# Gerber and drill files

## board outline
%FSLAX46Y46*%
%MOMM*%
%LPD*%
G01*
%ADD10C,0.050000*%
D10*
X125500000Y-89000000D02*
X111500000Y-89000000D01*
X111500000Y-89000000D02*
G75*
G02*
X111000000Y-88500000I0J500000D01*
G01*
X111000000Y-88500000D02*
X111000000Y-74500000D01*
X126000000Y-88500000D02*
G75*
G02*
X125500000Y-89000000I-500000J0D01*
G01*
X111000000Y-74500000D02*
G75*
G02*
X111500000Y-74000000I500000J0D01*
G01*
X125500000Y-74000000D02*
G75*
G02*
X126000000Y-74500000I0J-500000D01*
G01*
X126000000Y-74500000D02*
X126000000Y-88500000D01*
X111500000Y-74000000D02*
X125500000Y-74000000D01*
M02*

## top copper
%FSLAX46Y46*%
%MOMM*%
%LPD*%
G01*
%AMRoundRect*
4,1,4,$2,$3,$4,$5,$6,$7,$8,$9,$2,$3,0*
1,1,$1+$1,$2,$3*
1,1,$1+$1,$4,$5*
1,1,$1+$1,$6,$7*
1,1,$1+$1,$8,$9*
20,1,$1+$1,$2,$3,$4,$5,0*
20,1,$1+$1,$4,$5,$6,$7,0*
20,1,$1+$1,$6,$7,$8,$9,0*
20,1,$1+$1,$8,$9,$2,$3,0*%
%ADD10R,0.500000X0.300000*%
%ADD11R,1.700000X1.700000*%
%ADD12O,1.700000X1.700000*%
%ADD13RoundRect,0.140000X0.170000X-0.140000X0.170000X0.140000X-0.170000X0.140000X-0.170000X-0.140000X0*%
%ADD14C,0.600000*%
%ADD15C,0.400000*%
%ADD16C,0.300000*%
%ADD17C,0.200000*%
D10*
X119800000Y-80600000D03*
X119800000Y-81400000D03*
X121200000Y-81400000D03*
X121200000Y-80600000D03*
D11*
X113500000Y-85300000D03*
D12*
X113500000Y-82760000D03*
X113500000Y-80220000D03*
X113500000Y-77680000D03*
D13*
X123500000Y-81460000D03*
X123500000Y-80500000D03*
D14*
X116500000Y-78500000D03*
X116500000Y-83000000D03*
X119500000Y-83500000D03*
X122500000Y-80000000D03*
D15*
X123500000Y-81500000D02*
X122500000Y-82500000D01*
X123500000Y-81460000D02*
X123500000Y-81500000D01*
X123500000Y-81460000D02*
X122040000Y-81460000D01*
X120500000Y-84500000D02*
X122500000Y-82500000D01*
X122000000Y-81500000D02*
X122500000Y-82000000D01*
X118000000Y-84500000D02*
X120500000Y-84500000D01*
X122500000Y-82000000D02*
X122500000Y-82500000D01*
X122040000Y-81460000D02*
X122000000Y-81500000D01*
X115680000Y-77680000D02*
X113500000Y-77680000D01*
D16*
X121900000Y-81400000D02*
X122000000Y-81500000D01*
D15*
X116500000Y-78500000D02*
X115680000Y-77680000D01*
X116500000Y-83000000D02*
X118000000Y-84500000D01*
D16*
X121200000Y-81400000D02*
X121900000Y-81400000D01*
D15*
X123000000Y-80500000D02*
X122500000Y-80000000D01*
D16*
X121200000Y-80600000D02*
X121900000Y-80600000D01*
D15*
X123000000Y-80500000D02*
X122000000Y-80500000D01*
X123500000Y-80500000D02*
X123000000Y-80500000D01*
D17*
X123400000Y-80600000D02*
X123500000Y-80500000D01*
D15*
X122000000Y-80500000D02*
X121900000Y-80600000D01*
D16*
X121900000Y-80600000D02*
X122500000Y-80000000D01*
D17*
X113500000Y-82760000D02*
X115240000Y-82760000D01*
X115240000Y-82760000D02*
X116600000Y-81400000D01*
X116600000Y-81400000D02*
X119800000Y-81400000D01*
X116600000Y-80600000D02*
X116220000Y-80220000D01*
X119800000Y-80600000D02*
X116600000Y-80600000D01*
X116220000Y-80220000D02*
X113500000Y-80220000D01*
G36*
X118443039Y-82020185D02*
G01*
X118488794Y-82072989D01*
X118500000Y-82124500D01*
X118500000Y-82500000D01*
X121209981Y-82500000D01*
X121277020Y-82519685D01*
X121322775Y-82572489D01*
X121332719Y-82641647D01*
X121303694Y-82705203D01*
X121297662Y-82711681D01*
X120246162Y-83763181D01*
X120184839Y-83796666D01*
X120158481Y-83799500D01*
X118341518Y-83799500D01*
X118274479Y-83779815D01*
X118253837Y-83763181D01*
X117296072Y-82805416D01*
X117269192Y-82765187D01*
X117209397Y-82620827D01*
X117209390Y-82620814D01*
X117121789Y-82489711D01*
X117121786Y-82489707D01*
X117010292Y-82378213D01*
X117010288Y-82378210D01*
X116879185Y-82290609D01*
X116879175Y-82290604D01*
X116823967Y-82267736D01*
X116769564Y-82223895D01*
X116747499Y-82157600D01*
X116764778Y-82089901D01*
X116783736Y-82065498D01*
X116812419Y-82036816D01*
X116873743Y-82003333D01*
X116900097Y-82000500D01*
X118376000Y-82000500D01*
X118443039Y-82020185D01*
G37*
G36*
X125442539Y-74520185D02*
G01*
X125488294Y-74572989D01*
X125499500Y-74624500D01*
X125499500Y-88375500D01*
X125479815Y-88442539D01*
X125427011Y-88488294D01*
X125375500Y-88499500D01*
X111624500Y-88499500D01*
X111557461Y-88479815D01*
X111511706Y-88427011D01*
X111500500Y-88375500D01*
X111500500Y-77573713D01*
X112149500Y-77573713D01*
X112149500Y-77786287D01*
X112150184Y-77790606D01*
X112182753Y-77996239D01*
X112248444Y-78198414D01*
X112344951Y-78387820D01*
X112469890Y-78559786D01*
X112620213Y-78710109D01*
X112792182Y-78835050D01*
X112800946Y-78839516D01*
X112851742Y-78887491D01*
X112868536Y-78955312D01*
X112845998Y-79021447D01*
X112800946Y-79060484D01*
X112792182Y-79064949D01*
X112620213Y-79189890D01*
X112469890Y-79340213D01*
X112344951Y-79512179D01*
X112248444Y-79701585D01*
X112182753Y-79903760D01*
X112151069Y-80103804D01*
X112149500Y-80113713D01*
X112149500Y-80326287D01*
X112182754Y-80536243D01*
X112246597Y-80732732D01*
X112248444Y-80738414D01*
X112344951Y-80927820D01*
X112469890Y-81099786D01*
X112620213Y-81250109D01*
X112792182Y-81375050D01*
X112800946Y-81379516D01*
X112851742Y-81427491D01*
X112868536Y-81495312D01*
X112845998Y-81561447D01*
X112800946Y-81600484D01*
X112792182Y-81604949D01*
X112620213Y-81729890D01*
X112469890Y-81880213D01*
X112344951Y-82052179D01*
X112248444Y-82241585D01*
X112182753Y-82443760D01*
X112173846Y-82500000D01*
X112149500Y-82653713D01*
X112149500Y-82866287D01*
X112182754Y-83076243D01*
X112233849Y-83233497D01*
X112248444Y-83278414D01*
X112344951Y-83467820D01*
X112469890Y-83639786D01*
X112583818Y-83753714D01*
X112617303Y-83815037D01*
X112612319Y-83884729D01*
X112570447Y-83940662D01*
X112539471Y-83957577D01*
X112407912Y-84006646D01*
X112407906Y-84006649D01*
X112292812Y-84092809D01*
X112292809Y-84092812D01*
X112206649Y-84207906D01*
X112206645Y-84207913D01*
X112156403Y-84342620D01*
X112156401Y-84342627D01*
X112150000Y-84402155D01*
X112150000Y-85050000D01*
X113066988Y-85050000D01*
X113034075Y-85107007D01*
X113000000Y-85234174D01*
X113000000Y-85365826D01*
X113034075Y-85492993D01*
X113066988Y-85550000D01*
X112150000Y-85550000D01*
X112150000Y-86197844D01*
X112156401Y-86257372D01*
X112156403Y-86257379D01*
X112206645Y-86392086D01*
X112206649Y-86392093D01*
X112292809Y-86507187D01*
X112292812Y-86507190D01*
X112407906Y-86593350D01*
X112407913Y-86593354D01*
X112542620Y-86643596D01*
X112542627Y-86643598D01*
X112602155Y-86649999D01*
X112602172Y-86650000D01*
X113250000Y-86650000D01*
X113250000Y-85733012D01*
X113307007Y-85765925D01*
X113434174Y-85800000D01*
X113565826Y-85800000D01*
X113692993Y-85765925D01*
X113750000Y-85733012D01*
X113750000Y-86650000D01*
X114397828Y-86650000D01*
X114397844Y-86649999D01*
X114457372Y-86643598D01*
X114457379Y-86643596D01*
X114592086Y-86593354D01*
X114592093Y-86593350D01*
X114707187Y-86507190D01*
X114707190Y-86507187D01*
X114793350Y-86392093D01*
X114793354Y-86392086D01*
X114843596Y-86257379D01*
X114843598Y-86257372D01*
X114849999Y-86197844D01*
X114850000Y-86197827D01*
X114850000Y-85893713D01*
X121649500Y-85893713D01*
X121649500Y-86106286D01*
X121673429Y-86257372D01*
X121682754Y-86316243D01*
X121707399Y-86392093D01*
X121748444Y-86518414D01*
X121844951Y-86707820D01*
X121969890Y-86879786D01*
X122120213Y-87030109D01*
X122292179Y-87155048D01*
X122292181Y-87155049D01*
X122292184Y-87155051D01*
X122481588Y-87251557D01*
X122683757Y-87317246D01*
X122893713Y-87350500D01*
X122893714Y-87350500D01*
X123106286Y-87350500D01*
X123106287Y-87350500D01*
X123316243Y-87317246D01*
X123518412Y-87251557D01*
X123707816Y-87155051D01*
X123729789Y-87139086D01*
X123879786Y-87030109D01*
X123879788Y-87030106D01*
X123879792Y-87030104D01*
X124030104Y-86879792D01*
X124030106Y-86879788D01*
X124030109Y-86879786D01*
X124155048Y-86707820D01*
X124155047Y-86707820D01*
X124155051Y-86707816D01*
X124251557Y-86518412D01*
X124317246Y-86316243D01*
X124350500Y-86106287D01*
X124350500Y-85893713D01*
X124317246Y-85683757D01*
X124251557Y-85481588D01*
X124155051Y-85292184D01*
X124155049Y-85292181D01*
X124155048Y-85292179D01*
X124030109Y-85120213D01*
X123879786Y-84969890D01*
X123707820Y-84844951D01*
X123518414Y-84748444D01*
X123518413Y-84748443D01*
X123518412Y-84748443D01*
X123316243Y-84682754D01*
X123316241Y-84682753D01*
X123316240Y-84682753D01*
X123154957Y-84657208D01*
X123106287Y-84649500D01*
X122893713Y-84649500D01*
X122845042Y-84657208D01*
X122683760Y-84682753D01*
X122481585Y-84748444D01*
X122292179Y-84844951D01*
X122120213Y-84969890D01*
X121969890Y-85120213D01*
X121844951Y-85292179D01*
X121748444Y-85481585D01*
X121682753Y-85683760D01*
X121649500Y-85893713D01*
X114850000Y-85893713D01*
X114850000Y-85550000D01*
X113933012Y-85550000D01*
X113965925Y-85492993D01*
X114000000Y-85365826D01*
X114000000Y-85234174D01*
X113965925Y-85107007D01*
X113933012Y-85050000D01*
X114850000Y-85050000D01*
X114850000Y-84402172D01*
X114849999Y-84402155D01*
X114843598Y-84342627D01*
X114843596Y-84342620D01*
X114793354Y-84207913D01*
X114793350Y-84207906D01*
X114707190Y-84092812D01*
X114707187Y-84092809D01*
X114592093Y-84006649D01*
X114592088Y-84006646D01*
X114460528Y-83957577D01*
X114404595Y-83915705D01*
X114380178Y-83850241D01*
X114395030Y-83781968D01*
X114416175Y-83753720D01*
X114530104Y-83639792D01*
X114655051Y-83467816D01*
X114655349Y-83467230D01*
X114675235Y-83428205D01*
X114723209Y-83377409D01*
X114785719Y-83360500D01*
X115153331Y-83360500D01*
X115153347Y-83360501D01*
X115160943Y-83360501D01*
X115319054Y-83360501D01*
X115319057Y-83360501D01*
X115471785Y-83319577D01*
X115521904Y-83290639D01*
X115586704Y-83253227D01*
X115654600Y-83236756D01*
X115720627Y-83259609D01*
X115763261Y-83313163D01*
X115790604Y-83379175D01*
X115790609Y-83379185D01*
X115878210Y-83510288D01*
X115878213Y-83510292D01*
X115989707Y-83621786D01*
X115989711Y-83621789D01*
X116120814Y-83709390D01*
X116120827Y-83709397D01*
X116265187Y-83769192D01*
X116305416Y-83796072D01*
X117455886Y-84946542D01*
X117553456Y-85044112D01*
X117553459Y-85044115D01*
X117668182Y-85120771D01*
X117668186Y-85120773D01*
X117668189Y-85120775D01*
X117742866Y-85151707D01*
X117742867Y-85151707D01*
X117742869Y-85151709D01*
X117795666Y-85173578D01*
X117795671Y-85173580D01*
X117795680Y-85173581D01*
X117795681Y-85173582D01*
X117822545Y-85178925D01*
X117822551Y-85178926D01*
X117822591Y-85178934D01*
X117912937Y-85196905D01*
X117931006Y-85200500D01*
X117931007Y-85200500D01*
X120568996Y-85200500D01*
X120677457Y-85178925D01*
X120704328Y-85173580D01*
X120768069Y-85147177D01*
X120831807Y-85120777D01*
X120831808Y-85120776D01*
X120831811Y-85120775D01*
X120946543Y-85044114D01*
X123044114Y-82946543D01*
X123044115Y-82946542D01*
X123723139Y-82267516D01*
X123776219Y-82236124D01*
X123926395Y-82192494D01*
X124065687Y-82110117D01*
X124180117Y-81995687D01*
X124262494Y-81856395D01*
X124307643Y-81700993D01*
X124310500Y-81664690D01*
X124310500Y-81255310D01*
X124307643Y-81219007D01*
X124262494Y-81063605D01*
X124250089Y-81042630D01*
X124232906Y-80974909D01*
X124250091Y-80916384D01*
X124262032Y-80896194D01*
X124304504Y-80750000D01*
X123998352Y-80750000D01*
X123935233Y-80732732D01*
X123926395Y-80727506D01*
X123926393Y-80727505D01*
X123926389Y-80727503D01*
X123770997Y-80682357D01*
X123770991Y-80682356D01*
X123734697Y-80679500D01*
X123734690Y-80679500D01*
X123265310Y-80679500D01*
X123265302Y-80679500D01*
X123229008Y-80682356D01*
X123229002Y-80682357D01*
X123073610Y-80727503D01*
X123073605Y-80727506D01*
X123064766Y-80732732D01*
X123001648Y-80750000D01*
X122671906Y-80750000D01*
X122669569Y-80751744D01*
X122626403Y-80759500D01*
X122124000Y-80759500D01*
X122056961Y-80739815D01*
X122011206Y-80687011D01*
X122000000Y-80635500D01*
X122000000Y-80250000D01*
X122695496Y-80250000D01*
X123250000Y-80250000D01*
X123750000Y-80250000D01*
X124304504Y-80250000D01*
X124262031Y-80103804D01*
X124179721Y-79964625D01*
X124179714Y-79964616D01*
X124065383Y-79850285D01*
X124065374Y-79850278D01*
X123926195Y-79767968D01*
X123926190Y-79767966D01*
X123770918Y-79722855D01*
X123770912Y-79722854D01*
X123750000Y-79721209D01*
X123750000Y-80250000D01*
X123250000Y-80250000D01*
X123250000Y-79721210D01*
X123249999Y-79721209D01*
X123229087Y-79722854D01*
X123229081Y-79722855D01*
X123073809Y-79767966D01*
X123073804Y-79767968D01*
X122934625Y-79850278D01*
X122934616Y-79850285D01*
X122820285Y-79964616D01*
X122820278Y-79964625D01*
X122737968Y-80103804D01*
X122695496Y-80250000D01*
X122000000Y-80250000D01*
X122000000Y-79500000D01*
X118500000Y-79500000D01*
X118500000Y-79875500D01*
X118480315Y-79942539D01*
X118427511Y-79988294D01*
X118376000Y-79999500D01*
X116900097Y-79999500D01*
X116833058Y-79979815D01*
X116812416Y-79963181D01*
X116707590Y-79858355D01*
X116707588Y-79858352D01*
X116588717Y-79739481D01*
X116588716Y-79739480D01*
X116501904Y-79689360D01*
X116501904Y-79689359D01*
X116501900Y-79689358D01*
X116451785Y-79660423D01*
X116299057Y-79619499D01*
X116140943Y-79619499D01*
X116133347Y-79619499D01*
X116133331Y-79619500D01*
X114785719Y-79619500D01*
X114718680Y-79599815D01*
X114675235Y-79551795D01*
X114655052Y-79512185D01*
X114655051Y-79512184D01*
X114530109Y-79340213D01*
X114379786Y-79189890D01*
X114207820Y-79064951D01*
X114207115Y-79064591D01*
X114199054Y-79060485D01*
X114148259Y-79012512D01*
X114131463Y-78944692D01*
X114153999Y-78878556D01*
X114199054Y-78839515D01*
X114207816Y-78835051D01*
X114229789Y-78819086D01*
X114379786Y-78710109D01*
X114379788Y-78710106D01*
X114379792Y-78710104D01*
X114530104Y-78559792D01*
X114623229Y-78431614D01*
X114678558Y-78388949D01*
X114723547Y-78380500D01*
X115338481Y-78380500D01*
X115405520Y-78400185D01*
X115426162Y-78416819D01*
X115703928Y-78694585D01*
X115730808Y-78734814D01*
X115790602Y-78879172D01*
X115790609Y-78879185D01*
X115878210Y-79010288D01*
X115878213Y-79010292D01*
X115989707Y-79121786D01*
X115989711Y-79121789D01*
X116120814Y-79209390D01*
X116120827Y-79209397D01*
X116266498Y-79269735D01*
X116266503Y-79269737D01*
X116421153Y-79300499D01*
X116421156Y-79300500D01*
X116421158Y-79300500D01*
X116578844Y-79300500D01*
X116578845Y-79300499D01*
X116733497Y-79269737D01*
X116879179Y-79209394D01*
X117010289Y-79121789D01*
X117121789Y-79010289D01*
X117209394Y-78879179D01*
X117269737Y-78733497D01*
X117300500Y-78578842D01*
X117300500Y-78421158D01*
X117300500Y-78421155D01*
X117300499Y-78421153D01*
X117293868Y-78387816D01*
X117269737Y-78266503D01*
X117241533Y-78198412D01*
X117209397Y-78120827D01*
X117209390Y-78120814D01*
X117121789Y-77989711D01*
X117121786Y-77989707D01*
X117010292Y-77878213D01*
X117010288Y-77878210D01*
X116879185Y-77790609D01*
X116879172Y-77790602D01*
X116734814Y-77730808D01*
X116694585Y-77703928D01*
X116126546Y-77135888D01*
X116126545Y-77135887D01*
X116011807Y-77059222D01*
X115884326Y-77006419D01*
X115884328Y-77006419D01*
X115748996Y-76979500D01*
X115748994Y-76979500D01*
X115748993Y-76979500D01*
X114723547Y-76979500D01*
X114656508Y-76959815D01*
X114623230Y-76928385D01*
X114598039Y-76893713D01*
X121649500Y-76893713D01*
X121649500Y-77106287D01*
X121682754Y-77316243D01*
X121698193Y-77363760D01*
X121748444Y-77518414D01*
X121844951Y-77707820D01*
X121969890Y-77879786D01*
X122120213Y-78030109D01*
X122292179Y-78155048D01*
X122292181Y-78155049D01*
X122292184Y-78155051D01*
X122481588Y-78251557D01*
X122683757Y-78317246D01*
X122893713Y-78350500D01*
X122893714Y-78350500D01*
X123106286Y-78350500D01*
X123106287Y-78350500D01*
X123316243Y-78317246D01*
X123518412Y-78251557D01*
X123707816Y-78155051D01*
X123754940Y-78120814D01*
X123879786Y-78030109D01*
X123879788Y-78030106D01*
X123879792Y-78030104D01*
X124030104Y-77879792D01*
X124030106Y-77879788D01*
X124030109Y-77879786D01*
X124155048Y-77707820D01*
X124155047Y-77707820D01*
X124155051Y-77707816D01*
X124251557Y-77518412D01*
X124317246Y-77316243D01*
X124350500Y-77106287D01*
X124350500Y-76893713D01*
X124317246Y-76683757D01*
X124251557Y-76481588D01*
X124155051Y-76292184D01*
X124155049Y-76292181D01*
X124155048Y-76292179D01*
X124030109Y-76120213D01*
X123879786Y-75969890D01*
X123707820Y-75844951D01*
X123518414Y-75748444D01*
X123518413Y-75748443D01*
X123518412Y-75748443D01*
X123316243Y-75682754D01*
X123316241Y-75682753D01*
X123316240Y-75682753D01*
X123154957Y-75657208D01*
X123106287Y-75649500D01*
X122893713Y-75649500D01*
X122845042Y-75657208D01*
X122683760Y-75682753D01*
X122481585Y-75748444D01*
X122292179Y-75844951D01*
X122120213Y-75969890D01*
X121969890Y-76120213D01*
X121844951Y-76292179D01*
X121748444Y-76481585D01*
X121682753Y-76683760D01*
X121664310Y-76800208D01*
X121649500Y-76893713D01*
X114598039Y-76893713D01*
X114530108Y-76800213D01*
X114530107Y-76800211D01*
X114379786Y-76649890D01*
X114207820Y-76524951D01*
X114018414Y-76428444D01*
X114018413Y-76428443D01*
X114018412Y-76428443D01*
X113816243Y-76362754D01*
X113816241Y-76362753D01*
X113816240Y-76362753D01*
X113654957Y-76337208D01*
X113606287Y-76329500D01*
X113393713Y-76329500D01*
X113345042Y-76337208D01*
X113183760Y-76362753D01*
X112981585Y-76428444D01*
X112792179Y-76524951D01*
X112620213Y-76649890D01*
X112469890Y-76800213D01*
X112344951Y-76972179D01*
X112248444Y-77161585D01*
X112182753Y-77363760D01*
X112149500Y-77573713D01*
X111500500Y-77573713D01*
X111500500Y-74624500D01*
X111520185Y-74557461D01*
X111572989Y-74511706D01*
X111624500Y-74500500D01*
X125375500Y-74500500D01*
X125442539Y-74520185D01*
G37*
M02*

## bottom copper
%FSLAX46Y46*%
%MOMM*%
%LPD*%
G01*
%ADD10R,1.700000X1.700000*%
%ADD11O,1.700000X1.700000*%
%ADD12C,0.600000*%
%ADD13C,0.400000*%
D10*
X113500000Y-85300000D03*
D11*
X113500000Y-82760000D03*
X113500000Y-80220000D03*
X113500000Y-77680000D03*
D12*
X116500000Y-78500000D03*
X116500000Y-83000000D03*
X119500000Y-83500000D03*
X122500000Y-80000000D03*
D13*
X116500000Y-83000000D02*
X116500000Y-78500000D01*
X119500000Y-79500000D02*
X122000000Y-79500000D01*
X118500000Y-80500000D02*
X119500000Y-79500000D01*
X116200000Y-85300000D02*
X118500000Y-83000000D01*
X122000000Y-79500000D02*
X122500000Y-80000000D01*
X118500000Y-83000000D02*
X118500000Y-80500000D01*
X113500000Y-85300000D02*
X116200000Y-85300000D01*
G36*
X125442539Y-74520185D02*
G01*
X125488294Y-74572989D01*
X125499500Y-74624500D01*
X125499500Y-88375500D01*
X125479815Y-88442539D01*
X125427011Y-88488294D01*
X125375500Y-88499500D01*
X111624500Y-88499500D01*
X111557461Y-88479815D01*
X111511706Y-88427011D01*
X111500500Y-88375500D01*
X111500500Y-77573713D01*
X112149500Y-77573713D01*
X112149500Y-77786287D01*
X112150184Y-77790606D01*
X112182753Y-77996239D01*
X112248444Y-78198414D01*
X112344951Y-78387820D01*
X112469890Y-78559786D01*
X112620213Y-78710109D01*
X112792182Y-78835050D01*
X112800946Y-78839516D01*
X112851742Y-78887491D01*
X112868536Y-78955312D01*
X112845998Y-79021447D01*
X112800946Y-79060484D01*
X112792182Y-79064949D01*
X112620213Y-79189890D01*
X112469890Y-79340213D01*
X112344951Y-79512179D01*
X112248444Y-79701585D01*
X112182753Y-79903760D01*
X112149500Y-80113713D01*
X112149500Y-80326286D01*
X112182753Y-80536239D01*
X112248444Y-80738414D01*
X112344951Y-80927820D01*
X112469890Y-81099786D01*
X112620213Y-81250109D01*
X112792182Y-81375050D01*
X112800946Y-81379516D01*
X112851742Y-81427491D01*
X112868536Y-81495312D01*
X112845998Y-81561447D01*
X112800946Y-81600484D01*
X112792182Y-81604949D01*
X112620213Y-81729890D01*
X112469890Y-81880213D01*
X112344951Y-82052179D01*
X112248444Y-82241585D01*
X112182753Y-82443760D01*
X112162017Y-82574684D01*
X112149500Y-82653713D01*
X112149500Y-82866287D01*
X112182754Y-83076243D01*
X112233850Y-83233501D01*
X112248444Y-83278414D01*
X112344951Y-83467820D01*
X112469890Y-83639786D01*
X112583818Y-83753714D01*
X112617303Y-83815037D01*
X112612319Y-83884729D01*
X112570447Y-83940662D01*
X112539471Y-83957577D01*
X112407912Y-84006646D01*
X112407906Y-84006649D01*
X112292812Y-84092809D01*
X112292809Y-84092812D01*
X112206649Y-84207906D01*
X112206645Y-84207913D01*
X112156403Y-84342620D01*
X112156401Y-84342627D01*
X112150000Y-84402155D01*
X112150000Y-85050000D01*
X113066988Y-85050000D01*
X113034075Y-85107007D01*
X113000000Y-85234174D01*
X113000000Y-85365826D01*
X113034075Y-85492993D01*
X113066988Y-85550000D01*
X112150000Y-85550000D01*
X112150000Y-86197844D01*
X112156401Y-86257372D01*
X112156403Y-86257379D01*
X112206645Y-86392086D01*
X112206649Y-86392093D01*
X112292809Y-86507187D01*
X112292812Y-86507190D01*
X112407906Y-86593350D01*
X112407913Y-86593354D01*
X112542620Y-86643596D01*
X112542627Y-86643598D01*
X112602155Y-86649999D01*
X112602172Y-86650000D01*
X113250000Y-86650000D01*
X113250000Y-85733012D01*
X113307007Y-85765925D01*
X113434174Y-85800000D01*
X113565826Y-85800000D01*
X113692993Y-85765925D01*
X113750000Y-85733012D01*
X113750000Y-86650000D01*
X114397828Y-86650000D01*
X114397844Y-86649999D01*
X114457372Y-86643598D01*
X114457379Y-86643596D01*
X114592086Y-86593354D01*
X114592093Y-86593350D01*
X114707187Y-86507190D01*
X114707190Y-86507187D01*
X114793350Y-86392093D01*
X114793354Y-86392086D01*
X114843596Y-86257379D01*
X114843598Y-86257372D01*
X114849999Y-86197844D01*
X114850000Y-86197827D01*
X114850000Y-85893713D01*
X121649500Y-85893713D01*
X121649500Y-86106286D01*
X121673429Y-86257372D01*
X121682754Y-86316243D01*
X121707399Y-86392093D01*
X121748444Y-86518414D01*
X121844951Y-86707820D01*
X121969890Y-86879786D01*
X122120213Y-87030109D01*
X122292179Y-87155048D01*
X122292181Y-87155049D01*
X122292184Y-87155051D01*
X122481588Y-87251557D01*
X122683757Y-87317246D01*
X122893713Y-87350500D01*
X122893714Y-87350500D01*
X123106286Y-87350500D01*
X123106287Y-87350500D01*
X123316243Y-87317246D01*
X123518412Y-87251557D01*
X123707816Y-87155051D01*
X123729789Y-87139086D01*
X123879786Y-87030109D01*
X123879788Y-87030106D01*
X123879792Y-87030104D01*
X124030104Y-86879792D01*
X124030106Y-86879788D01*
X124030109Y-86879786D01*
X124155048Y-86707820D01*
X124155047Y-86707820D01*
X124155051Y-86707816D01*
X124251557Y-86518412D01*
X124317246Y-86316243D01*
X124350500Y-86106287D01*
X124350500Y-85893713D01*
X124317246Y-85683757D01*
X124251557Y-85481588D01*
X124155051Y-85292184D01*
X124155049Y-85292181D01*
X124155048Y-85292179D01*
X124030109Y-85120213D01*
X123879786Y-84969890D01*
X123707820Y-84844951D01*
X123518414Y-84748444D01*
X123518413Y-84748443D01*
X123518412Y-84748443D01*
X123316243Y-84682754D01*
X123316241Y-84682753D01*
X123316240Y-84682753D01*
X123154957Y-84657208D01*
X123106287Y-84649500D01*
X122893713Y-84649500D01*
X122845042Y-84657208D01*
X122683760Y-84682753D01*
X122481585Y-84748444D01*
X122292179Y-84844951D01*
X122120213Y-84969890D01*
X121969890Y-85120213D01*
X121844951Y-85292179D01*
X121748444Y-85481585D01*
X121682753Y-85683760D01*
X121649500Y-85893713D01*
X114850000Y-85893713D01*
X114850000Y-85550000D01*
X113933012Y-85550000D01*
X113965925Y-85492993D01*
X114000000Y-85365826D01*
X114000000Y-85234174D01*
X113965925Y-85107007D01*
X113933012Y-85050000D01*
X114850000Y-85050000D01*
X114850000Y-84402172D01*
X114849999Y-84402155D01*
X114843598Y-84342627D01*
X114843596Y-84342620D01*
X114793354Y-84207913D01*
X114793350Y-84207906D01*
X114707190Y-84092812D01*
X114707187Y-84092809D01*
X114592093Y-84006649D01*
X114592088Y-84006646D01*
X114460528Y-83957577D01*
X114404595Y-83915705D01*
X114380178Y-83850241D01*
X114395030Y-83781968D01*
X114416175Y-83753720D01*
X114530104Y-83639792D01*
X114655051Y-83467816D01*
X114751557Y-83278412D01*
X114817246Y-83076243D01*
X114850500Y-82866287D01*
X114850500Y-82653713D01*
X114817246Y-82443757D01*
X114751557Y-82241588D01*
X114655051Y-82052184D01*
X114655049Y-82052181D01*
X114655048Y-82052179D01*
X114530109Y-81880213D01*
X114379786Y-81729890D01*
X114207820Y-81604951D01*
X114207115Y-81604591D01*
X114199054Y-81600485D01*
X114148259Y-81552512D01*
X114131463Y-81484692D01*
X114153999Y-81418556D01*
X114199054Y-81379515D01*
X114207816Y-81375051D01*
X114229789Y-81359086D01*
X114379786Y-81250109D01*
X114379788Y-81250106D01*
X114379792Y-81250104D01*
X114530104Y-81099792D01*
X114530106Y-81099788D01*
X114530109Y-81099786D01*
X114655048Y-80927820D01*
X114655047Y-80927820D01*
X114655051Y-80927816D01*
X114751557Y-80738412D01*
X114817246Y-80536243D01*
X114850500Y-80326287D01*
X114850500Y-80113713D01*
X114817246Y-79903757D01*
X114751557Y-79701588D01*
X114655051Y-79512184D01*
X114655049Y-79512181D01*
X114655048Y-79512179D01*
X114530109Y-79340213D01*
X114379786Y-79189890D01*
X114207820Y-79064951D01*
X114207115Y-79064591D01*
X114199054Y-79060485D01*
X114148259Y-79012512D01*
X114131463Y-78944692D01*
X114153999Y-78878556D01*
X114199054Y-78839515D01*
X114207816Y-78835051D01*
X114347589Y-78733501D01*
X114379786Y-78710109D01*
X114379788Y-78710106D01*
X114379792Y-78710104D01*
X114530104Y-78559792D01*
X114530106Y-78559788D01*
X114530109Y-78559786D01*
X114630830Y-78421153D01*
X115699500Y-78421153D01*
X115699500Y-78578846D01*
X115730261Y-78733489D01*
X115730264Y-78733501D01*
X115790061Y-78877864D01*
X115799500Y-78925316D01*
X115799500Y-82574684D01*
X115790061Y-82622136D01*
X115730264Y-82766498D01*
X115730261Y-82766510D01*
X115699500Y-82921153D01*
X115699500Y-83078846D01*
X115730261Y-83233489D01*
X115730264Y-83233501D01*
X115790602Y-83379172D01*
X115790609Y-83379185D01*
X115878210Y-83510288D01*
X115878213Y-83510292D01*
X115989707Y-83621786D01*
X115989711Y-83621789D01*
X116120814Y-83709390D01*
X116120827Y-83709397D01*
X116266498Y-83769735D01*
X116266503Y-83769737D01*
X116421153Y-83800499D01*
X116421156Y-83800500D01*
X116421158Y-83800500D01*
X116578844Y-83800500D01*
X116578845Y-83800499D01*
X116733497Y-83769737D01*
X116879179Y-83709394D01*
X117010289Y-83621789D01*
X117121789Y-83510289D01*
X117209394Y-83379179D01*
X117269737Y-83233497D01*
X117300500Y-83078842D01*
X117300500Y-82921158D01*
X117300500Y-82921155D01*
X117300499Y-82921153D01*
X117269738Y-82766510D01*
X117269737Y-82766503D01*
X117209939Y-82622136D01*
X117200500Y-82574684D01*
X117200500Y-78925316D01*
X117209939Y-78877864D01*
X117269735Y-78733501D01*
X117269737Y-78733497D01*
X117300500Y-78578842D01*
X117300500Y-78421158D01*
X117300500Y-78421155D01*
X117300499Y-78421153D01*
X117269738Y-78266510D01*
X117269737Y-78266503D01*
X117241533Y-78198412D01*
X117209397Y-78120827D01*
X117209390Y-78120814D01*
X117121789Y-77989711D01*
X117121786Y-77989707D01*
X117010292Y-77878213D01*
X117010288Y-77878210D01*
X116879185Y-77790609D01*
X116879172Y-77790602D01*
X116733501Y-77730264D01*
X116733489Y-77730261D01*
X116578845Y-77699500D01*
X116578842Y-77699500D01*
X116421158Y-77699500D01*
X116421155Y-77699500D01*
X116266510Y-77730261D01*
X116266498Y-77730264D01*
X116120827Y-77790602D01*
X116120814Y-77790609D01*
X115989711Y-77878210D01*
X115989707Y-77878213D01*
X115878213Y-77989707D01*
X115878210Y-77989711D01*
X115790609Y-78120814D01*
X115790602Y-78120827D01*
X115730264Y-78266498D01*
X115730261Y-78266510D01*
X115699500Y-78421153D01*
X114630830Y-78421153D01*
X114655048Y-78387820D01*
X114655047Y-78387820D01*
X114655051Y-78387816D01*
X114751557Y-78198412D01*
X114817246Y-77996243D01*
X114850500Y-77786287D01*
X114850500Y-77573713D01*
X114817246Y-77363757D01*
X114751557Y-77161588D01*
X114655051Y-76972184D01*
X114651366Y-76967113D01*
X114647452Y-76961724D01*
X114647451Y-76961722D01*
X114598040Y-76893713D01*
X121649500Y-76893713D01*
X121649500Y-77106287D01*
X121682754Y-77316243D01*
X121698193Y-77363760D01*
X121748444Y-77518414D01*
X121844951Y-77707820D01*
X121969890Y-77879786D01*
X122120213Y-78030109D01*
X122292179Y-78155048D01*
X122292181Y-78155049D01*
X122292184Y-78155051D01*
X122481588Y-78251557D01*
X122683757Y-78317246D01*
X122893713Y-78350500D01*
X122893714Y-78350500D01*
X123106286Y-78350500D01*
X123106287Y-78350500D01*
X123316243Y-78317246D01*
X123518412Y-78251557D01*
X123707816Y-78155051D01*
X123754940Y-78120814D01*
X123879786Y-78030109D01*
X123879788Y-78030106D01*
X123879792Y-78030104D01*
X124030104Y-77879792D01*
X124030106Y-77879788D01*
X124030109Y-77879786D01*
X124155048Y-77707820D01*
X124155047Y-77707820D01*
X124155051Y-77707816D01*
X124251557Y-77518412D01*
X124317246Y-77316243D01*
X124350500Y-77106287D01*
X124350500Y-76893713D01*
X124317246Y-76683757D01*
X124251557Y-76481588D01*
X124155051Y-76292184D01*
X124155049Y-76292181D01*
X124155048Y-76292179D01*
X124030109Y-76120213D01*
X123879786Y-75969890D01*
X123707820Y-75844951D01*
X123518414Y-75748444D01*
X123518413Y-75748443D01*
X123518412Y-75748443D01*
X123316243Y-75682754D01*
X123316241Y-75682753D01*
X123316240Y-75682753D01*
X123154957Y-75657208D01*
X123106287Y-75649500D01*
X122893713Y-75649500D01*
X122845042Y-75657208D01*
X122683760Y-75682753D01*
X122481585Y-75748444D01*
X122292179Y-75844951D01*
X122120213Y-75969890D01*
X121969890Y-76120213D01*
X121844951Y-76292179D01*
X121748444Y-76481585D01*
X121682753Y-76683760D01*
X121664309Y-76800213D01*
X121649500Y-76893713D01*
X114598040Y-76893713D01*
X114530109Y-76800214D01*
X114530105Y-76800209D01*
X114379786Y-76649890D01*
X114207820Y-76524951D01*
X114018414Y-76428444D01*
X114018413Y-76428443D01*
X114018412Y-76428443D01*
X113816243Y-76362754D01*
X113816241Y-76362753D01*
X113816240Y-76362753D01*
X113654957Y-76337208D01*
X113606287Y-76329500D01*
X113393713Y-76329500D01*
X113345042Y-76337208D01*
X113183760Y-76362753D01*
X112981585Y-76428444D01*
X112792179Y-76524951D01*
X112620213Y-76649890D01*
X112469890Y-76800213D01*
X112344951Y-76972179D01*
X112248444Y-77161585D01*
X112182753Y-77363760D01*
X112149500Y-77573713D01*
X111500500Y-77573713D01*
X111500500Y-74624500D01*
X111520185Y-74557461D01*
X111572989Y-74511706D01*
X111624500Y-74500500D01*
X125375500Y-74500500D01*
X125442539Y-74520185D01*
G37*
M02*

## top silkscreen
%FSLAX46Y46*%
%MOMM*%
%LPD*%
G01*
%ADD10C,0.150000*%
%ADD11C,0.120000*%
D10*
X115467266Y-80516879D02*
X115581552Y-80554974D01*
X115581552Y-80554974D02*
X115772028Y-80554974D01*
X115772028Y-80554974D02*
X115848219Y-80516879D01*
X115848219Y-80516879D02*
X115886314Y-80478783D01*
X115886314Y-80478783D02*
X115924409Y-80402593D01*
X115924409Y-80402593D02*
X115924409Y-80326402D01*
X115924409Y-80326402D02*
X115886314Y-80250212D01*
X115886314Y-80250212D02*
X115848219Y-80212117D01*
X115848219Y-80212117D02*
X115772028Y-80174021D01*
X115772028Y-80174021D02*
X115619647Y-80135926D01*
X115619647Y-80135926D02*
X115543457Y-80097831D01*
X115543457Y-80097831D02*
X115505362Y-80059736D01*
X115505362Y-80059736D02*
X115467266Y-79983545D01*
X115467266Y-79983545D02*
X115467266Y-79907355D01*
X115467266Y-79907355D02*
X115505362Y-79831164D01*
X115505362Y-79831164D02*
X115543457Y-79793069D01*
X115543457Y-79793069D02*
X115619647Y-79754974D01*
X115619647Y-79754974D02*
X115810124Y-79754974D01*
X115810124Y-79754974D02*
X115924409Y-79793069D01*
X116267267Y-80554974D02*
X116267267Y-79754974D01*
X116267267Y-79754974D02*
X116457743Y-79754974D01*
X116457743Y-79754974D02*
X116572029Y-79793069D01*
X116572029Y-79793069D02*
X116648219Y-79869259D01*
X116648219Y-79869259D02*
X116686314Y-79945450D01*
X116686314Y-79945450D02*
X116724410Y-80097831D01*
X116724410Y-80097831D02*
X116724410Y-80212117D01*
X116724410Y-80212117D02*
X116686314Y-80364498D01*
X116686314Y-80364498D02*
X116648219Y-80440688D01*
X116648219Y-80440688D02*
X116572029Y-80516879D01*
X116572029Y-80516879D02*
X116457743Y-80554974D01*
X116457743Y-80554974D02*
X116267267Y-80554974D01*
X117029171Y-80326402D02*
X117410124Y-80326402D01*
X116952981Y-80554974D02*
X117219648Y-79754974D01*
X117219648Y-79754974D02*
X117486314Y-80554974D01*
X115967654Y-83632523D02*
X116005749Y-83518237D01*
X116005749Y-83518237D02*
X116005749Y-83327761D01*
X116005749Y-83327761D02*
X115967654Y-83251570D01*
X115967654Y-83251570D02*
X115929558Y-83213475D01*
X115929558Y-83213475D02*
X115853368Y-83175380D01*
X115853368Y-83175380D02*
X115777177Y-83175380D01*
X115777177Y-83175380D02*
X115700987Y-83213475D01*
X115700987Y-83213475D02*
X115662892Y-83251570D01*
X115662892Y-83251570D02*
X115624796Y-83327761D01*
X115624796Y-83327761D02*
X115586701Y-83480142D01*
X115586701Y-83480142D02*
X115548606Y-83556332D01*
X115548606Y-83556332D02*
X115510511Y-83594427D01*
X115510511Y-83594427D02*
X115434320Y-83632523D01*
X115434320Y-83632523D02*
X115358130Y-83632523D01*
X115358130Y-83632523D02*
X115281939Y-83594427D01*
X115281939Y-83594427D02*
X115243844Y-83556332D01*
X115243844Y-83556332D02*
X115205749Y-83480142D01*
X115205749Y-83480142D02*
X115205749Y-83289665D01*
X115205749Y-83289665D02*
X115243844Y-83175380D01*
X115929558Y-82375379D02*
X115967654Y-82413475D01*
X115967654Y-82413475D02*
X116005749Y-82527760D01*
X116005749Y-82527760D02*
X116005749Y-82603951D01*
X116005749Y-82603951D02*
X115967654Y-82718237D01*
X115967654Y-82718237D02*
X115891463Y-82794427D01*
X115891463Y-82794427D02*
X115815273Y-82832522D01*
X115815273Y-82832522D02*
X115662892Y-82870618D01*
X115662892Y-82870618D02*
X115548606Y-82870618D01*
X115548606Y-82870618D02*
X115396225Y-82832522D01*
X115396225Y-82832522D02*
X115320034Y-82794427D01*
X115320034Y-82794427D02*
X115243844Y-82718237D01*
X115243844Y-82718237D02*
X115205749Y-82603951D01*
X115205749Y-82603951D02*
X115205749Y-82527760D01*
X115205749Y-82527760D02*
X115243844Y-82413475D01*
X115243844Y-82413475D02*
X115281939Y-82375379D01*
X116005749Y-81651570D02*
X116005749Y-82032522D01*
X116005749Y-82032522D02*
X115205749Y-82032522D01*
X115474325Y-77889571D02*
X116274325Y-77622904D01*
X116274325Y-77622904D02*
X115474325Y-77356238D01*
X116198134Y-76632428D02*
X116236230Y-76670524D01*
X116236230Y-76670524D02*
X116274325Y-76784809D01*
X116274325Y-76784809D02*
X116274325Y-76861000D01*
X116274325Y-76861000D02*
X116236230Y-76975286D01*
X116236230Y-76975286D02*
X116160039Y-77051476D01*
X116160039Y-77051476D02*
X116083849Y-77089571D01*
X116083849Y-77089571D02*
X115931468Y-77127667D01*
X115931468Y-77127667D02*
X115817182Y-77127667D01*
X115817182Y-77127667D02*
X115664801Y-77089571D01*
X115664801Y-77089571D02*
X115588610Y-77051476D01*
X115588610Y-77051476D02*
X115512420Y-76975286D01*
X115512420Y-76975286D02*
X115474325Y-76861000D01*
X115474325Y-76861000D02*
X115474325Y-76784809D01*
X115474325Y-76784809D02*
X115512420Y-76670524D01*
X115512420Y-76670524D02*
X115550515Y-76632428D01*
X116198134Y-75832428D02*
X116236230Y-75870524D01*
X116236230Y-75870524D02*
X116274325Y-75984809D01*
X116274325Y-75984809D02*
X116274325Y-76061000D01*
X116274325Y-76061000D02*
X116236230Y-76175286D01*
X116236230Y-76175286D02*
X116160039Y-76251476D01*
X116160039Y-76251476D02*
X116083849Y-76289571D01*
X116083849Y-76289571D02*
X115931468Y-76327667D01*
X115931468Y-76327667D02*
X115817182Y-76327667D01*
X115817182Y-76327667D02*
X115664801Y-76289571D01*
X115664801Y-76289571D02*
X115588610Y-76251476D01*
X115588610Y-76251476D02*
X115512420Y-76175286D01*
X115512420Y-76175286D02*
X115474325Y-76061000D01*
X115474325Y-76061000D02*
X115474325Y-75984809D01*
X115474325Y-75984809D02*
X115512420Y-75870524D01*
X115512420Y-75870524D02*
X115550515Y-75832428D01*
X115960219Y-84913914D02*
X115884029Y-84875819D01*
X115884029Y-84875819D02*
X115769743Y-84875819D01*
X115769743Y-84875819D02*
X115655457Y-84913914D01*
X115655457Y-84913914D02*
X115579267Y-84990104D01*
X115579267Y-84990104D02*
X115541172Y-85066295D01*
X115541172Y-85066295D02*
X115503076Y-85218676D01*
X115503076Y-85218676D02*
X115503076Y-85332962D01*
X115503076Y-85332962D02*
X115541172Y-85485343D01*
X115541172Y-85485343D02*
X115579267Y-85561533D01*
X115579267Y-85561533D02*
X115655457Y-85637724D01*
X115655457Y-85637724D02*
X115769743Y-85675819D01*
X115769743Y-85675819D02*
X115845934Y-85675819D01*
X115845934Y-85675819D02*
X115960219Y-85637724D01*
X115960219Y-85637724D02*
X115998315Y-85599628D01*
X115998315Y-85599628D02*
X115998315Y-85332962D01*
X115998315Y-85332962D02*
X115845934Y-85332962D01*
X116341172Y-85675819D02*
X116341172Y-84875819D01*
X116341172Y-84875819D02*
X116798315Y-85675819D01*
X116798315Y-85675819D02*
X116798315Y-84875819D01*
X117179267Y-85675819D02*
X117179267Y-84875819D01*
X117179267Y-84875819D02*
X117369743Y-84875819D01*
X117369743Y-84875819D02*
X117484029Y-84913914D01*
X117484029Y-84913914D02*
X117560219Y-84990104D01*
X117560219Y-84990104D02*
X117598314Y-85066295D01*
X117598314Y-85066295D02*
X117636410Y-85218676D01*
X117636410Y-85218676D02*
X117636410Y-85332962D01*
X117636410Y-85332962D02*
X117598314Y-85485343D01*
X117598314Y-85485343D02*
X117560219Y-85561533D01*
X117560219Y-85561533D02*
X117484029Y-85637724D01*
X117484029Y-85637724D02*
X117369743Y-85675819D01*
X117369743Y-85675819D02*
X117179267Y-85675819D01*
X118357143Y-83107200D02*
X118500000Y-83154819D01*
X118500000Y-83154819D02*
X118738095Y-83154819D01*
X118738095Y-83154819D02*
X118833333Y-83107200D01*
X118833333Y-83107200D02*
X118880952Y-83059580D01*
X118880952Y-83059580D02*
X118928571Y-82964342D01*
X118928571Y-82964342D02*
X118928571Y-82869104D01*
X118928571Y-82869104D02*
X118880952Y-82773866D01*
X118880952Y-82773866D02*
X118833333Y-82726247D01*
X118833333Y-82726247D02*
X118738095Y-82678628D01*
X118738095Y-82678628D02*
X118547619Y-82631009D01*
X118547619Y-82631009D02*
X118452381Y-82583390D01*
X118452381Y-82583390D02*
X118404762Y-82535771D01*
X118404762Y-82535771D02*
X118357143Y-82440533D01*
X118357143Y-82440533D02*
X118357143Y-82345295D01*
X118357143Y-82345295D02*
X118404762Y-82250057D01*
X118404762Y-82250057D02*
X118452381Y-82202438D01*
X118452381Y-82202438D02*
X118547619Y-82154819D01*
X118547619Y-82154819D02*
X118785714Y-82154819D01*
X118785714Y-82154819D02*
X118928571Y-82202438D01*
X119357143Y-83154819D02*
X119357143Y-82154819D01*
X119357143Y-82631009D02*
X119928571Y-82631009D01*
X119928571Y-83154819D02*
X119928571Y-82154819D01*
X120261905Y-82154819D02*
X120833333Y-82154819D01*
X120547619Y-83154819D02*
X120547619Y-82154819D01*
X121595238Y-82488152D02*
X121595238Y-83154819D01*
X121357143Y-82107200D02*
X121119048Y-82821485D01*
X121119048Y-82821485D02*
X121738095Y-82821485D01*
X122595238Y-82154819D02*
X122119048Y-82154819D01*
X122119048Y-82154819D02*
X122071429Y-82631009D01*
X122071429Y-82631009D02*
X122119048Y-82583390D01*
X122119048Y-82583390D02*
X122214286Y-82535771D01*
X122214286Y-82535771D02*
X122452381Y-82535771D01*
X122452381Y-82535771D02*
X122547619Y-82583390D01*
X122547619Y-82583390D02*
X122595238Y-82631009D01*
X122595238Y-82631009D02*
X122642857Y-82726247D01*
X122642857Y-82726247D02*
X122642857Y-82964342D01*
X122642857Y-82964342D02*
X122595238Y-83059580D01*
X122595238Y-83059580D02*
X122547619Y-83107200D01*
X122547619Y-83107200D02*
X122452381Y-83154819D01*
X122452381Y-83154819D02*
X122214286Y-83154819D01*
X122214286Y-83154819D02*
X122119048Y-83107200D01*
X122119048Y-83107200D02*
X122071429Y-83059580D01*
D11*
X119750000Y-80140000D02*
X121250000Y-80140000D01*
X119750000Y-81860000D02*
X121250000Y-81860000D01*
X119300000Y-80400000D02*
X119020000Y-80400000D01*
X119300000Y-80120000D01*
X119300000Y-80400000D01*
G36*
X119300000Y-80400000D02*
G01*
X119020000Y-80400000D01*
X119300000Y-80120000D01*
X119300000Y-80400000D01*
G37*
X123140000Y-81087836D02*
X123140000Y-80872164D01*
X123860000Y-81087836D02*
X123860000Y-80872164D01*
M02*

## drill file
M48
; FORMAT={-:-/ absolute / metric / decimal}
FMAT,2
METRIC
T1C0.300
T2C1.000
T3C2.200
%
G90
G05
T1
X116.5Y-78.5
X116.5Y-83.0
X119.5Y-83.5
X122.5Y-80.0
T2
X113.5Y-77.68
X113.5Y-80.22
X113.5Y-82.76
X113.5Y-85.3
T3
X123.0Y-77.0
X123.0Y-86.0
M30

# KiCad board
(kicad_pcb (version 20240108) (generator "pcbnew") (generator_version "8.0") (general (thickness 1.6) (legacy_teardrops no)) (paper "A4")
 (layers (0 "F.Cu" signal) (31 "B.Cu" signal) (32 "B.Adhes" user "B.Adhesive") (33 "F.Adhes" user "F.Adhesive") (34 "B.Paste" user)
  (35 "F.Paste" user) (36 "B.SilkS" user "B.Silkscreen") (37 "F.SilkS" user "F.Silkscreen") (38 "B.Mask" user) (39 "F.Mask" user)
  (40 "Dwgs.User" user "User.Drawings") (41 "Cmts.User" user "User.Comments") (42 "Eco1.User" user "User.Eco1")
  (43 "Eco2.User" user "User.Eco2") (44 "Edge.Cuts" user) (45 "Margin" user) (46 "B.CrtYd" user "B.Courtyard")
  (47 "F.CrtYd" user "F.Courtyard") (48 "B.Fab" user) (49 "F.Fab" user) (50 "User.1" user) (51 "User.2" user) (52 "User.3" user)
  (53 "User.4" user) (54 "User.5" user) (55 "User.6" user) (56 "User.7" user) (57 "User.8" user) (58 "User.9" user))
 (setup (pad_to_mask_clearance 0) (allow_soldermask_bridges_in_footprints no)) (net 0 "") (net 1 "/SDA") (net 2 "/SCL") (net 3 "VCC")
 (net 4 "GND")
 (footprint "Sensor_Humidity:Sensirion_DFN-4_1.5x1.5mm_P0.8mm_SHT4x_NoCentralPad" (layer "F.Cu") (at 120.5 81)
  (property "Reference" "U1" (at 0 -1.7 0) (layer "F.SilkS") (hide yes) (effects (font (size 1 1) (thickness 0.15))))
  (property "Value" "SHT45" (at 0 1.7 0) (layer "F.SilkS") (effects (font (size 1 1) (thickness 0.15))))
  (fp_line (start -0.75 -0.86) (end 0.75 -0.86) (stroke (width 0.12) (type solid)) (layer "F.SilkS"))
  (fp_line (start -0.75 0.86) (end 0.75 0.86) (stroke (width 0.12) (type solid)) (layer "F.SilkS"))
  (fp_poly
   (pts (xy -1.2 -0.6) (xy -1.48 -0.6) (xy -1.2 -0.88) (xy -1.2 -0.6)) (stroke (width 0.12) (type solid)) (fill solid) (layer "F.SilkS"))
  (pad "1" smd rect (at -0.7 -0.4) (size 0.5 0.3) (layers "F.Cu" "F.Paste" "F.Mask") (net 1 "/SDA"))
  (pad "2" smd rect (at -0.7 0.4) (size 0.5 0.3) (layers "F.Cu" "F.Paste" "F.Mask") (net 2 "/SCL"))
  (pad "3" smd rect (at 0.7 0.4) (size 0.5 0.3) (layers "F.Cu" "F.Paste" "F.Mask") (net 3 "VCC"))
  (pad "4" smd rect (at 0.7 -0.4) (size 0.5 0.3) (layers "F.Cu" "F.Paste" "F.Mask") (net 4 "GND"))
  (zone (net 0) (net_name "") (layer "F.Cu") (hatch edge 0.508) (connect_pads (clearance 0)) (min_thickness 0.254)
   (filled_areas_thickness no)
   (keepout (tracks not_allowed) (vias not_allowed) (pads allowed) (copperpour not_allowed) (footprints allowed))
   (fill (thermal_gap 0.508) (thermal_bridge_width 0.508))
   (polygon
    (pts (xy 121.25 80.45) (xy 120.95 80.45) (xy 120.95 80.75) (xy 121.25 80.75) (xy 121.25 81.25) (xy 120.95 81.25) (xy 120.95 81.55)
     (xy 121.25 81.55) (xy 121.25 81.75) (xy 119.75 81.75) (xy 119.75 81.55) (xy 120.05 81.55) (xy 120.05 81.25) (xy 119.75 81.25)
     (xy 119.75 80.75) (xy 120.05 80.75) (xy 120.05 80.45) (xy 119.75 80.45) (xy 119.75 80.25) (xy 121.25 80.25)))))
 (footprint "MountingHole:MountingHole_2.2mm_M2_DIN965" (layer "F.Cu") (at 123 86)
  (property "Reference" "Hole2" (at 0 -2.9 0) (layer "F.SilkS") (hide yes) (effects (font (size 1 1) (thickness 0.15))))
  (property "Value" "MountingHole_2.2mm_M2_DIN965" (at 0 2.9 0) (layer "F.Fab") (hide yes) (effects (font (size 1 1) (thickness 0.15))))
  (pad "" np_thru_hole circle (at 0 0) (size 2.2 2.2) (drill 2.2) (layers "*.Cu" "*.Mask")))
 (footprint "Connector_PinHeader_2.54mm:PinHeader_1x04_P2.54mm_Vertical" (layer "F.Cu") (at 113.5 85.3 180)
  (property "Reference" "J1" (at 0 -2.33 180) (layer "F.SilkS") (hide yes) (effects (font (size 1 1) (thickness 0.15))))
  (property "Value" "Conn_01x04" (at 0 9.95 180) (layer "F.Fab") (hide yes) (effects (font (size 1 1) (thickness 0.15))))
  (pad "1" thru_hole rect (at 0 0 180) (size 1.7 1.7) (drill 1) (layers "*.Cu" "*.Mask") (remove_unused_layers no) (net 4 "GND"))
  (pad "2" thru_hole oval (at 0 2.54 180) (size 1.7 1.7) (drill 1) (layers "*.Cu" "*.Mask") (remove_unused_layers no) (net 2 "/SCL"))
  (pad "3" thru_hole oval (at 0 5.08 180) (size 1.7 1.7) (drill 1) (layers "*.Cu" "*.Mask") (remove_unused_layers no) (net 1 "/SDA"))
  (pad "4" thru_hole oval (at 0 7.62 180) (size 1.7 1.7) (drill 1) (layers "*.Cu" "*.Mask") (remove_unused_layers no) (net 3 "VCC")))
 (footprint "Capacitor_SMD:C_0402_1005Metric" (layer "F.Cu") (at 123.5 80.98 90)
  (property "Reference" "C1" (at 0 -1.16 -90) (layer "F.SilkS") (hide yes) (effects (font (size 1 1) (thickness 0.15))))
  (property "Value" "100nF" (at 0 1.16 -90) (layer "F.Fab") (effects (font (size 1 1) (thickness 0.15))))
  (fp_line (start -0.107836 -0.36) (end 0.107836 -0.36) (stroke (width 0.12) (type solid)) (layer "F.SilkS"))
  (fp_line (start -0.107836 0.36) (end 0.107836 0.36) (stroke (width 0.12) (type solid)) (layer "F.SilkS"))
  (pad "1" smd roundrect (at -0.48 0 90) (size 0.56 0.62) (layers "F.Cu" "F.Paste" "F.Mask") (roundrect_rratio 0.25) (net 3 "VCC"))
  (pad "2" smd roundrect (at 0.48 0 90) (size 0.56 0.62) (layers "F.Cu" "F.Paste" "F.Mask") (roundrect_rratio 0.25) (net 4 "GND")))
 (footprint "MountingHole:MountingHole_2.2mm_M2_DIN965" (layer "F.Cu") (at 123 77)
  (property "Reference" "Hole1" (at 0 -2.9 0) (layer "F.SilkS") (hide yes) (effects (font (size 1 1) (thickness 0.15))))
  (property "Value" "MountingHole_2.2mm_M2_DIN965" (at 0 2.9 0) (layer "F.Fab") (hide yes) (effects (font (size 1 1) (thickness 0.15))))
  (pad "" np_thru_hole circle (at 0 0) (size 2.2 2.2) (drill 2.2) (layers "*.Cu" "*.Mask")))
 (gr_line (start 125.5 89) (end 111.5 89) (stroke (width 0.05) (type default)) (layer "Edge.Cuts"))
 (gr_arc (start 111.5 89) (mid 111.146447 88.853553) (end 111 88.5) (stroke (width 0.05) (type default)) (layer "Edge.Cuts"))
 (gr_line (start 111 88.5) (end 111 74.5) (stroke (width 0.05) (type default)) (layer "Edge.Cuts"))
 (gr_arc (start 126 88.5) (mid 125.853553 88.853553) (end 125.5 89) (stroke (width 0.05) (type default)) (layer "Edge.Cuts"))
 (gr_arc (start 111 74.5) (mid 111.146447 74.146447) (end 111.5 74) (stroke (width 0.05) (type default)) (layer "Edge.Cuts"))
 (gr_arc (start 125.5 74) (mid 125.853553 74.146447) (end 126 74.5) (stroke (width 0.05) (type default)) (layer "Edge.Cuts"))
 (gr_line (start 126 74.5) (end 126 88.5) (stroke (width 0.05) (type default)) (layer "Edge.Cuts"))
 (gr_line (start 111.5 74) (end 125.5 74) (stroke (width 0.05) (type default)) (layer "Edge.Cuts"))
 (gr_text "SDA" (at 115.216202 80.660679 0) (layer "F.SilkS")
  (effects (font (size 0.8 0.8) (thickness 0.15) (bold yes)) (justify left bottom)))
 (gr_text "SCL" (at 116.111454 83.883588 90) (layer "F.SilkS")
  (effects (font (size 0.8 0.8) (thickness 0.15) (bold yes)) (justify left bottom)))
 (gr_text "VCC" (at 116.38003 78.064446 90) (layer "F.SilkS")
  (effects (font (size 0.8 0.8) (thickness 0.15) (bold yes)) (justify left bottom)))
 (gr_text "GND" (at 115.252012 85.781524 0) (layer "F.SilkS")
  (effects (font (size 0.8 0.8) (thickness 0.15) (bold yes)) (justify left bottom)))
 (segment (start 123.5 81.5) (end 122.5 82.5) (width 0.4) (layer "F.Cu") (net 3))
 (segment (start 123.5 81.46) (end 123.5 81.5) (width 0.4) (layer "F.Cu") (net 3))
 (segment (start 123.5 81.46) (end 122.04 81.46) (width 0.4) (layer "F.Cu") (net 3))
 (segment (start 120.5 84.5) (end 122.5 82.5) (width 0.4) (layer "F.Cu") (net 3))
 (segment (start 122 81.5) (end 122.5 82) (width 0.4) (layer "F.Cu") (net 3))
 (segment (start 118 84.5) (end 120.5 84.5) (width 0.4) (layer "F.Cu") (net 3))
 (segment (start 122.5 82) (end 122.5 82.5) (width 0.4) (layer "F.Cu") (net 3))
 (segment (start 122.04 81.46) (end 122 81.5) (width 0.4) (layer "F.Cu") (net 3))
 (segment (start 115.68 77.68) (end 113.5 77.68) (width 0.4) (layer "F.Cu") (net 3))
 (segment (start 121.9 81.4) (end 122 81.5) (width 0.3) (layer "F.Cu") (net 3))
 (segment (start 116.5 78.5) (end 115.68 77.68) (width 0.4) (layer "F.Cu") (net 3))
 (segment (start 116.5 83) (end 118 84.5) (width 0.4) (layer "F.Cu") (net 3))
 (segment (start 121.2 81.4) (end 121.9 81.4) (width 0.3) (layer "F.Cu") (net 3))
 (via (at 116.5 78.5) (size 0.6) (drill 0.3) (layers "F.Cu" "B.Cu") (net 3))
 (via (at 116.5 83) (size 0.6) (drill 0.3) (layers "F.Cu" "B.Cu") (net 3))
 (segment (start 116.5 83) (end 116.5 78.5) (width 0.4) (layer "B.Cu") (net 3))
 (segment (start 123 80.5) (end 122.5 80) (width 0.4) (layer "F.Cu") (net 4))
 (segment (start 121.2 80.6) (end 121.9 80.6) (width 0.3) (layer "F.Cu") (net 4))
 (segment (start 123 80.5) (end 122 80.5) (width 0.4) (layer "F.Cu") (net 4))
 (segment (start 123.5 80.5) (end 123 80.5) (width 0.4) (layer "F.Cu") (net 4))
 (segment (start 123.4 80.6) (end 123.5 80.5) (width 0.2) (layer "F.Cu") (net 4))
 (segment (start 122 80.5) (end 121.9 80.6) (width 0.4) (layer "F.Cu") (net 4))
 (segment (start 121.9 80.6) (end 122.5 80) (width 0.3) (layer "F.Cu") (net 4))
 (via (at 119.5 83.5) (size 0.6) (drill 0.3) (layers "F.Cu" "B.Cu") (free yes) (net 4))
 (via (at 122.5 80) (size 0.6) (drill 0.3) (layers "F.Cu" "B.Cu") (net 4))
 (segment (start 119.5 79.5) (end 122 79.5) (width 0.4) (layer "B.Cu") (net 4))
 (segment (start 118.5 80.5) (end 119.5 79.5) (width 0.4) (layer "B.Cu") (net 4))
 (segment (start 116.2 85.3) (end 118.5 83) (width 0.4) (layer "B.Cu") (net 4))
 (segment (start 122 79.5) (end 122.5 80) (width 0.4) (layer "B.Cu") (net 4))
 (segment (start 118.5 83) (end 118.5 80.5) (width 0.4) (layer "B.Cu") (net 4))
 (segment (start 113.5 85.3) (end 116.2 85.3) (width 0.4) (layer "B.Cu") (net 4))
 (segment (start 113.5 82.76) (end 115.24 82.76) (width 0.2) (layer "F.Cu") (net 2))
 (segment (start 115.24 82.76) (end 116.6 81.4) (width 0.2) (layer "F.Cu") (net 2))
 (segment (start 116.6 81.4) (end 119.8 81.4) (width 0.2) (layer "F.Cu") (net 2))
 (segment (start 116.6 80.6) (end 116.22 80.22) (width 0.2) (layer "F.Cu") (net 1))
 (segment (start 119.8 80.6) (end 116.6 80.6) (width 0.2) (layer "F.Cu") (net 1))
 (segment (start 116.22 80.22) (end 113.5 80.22) (width 0.2) (layer "F.Cu") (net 1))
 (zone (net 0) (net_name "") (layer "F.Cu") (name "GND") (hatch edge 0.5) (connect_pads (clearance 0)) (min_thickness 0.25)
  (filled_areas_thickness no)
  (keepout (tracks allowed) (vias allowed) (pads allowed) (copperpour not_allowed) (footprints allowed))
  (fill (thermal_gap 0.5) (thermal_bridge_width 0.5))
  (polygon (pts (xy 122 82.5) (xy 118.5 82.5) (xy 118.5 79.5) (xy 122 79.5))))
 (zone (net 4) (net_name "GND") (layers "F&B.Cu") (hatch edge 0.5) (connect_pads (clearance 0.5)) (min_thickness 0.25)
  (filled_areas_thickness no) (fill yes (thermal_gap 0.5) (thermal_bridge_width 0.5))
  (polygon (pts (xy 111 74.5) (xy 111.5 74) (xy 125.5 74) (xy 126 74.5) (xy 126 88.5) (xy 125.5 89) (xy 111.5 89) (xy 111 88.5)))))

